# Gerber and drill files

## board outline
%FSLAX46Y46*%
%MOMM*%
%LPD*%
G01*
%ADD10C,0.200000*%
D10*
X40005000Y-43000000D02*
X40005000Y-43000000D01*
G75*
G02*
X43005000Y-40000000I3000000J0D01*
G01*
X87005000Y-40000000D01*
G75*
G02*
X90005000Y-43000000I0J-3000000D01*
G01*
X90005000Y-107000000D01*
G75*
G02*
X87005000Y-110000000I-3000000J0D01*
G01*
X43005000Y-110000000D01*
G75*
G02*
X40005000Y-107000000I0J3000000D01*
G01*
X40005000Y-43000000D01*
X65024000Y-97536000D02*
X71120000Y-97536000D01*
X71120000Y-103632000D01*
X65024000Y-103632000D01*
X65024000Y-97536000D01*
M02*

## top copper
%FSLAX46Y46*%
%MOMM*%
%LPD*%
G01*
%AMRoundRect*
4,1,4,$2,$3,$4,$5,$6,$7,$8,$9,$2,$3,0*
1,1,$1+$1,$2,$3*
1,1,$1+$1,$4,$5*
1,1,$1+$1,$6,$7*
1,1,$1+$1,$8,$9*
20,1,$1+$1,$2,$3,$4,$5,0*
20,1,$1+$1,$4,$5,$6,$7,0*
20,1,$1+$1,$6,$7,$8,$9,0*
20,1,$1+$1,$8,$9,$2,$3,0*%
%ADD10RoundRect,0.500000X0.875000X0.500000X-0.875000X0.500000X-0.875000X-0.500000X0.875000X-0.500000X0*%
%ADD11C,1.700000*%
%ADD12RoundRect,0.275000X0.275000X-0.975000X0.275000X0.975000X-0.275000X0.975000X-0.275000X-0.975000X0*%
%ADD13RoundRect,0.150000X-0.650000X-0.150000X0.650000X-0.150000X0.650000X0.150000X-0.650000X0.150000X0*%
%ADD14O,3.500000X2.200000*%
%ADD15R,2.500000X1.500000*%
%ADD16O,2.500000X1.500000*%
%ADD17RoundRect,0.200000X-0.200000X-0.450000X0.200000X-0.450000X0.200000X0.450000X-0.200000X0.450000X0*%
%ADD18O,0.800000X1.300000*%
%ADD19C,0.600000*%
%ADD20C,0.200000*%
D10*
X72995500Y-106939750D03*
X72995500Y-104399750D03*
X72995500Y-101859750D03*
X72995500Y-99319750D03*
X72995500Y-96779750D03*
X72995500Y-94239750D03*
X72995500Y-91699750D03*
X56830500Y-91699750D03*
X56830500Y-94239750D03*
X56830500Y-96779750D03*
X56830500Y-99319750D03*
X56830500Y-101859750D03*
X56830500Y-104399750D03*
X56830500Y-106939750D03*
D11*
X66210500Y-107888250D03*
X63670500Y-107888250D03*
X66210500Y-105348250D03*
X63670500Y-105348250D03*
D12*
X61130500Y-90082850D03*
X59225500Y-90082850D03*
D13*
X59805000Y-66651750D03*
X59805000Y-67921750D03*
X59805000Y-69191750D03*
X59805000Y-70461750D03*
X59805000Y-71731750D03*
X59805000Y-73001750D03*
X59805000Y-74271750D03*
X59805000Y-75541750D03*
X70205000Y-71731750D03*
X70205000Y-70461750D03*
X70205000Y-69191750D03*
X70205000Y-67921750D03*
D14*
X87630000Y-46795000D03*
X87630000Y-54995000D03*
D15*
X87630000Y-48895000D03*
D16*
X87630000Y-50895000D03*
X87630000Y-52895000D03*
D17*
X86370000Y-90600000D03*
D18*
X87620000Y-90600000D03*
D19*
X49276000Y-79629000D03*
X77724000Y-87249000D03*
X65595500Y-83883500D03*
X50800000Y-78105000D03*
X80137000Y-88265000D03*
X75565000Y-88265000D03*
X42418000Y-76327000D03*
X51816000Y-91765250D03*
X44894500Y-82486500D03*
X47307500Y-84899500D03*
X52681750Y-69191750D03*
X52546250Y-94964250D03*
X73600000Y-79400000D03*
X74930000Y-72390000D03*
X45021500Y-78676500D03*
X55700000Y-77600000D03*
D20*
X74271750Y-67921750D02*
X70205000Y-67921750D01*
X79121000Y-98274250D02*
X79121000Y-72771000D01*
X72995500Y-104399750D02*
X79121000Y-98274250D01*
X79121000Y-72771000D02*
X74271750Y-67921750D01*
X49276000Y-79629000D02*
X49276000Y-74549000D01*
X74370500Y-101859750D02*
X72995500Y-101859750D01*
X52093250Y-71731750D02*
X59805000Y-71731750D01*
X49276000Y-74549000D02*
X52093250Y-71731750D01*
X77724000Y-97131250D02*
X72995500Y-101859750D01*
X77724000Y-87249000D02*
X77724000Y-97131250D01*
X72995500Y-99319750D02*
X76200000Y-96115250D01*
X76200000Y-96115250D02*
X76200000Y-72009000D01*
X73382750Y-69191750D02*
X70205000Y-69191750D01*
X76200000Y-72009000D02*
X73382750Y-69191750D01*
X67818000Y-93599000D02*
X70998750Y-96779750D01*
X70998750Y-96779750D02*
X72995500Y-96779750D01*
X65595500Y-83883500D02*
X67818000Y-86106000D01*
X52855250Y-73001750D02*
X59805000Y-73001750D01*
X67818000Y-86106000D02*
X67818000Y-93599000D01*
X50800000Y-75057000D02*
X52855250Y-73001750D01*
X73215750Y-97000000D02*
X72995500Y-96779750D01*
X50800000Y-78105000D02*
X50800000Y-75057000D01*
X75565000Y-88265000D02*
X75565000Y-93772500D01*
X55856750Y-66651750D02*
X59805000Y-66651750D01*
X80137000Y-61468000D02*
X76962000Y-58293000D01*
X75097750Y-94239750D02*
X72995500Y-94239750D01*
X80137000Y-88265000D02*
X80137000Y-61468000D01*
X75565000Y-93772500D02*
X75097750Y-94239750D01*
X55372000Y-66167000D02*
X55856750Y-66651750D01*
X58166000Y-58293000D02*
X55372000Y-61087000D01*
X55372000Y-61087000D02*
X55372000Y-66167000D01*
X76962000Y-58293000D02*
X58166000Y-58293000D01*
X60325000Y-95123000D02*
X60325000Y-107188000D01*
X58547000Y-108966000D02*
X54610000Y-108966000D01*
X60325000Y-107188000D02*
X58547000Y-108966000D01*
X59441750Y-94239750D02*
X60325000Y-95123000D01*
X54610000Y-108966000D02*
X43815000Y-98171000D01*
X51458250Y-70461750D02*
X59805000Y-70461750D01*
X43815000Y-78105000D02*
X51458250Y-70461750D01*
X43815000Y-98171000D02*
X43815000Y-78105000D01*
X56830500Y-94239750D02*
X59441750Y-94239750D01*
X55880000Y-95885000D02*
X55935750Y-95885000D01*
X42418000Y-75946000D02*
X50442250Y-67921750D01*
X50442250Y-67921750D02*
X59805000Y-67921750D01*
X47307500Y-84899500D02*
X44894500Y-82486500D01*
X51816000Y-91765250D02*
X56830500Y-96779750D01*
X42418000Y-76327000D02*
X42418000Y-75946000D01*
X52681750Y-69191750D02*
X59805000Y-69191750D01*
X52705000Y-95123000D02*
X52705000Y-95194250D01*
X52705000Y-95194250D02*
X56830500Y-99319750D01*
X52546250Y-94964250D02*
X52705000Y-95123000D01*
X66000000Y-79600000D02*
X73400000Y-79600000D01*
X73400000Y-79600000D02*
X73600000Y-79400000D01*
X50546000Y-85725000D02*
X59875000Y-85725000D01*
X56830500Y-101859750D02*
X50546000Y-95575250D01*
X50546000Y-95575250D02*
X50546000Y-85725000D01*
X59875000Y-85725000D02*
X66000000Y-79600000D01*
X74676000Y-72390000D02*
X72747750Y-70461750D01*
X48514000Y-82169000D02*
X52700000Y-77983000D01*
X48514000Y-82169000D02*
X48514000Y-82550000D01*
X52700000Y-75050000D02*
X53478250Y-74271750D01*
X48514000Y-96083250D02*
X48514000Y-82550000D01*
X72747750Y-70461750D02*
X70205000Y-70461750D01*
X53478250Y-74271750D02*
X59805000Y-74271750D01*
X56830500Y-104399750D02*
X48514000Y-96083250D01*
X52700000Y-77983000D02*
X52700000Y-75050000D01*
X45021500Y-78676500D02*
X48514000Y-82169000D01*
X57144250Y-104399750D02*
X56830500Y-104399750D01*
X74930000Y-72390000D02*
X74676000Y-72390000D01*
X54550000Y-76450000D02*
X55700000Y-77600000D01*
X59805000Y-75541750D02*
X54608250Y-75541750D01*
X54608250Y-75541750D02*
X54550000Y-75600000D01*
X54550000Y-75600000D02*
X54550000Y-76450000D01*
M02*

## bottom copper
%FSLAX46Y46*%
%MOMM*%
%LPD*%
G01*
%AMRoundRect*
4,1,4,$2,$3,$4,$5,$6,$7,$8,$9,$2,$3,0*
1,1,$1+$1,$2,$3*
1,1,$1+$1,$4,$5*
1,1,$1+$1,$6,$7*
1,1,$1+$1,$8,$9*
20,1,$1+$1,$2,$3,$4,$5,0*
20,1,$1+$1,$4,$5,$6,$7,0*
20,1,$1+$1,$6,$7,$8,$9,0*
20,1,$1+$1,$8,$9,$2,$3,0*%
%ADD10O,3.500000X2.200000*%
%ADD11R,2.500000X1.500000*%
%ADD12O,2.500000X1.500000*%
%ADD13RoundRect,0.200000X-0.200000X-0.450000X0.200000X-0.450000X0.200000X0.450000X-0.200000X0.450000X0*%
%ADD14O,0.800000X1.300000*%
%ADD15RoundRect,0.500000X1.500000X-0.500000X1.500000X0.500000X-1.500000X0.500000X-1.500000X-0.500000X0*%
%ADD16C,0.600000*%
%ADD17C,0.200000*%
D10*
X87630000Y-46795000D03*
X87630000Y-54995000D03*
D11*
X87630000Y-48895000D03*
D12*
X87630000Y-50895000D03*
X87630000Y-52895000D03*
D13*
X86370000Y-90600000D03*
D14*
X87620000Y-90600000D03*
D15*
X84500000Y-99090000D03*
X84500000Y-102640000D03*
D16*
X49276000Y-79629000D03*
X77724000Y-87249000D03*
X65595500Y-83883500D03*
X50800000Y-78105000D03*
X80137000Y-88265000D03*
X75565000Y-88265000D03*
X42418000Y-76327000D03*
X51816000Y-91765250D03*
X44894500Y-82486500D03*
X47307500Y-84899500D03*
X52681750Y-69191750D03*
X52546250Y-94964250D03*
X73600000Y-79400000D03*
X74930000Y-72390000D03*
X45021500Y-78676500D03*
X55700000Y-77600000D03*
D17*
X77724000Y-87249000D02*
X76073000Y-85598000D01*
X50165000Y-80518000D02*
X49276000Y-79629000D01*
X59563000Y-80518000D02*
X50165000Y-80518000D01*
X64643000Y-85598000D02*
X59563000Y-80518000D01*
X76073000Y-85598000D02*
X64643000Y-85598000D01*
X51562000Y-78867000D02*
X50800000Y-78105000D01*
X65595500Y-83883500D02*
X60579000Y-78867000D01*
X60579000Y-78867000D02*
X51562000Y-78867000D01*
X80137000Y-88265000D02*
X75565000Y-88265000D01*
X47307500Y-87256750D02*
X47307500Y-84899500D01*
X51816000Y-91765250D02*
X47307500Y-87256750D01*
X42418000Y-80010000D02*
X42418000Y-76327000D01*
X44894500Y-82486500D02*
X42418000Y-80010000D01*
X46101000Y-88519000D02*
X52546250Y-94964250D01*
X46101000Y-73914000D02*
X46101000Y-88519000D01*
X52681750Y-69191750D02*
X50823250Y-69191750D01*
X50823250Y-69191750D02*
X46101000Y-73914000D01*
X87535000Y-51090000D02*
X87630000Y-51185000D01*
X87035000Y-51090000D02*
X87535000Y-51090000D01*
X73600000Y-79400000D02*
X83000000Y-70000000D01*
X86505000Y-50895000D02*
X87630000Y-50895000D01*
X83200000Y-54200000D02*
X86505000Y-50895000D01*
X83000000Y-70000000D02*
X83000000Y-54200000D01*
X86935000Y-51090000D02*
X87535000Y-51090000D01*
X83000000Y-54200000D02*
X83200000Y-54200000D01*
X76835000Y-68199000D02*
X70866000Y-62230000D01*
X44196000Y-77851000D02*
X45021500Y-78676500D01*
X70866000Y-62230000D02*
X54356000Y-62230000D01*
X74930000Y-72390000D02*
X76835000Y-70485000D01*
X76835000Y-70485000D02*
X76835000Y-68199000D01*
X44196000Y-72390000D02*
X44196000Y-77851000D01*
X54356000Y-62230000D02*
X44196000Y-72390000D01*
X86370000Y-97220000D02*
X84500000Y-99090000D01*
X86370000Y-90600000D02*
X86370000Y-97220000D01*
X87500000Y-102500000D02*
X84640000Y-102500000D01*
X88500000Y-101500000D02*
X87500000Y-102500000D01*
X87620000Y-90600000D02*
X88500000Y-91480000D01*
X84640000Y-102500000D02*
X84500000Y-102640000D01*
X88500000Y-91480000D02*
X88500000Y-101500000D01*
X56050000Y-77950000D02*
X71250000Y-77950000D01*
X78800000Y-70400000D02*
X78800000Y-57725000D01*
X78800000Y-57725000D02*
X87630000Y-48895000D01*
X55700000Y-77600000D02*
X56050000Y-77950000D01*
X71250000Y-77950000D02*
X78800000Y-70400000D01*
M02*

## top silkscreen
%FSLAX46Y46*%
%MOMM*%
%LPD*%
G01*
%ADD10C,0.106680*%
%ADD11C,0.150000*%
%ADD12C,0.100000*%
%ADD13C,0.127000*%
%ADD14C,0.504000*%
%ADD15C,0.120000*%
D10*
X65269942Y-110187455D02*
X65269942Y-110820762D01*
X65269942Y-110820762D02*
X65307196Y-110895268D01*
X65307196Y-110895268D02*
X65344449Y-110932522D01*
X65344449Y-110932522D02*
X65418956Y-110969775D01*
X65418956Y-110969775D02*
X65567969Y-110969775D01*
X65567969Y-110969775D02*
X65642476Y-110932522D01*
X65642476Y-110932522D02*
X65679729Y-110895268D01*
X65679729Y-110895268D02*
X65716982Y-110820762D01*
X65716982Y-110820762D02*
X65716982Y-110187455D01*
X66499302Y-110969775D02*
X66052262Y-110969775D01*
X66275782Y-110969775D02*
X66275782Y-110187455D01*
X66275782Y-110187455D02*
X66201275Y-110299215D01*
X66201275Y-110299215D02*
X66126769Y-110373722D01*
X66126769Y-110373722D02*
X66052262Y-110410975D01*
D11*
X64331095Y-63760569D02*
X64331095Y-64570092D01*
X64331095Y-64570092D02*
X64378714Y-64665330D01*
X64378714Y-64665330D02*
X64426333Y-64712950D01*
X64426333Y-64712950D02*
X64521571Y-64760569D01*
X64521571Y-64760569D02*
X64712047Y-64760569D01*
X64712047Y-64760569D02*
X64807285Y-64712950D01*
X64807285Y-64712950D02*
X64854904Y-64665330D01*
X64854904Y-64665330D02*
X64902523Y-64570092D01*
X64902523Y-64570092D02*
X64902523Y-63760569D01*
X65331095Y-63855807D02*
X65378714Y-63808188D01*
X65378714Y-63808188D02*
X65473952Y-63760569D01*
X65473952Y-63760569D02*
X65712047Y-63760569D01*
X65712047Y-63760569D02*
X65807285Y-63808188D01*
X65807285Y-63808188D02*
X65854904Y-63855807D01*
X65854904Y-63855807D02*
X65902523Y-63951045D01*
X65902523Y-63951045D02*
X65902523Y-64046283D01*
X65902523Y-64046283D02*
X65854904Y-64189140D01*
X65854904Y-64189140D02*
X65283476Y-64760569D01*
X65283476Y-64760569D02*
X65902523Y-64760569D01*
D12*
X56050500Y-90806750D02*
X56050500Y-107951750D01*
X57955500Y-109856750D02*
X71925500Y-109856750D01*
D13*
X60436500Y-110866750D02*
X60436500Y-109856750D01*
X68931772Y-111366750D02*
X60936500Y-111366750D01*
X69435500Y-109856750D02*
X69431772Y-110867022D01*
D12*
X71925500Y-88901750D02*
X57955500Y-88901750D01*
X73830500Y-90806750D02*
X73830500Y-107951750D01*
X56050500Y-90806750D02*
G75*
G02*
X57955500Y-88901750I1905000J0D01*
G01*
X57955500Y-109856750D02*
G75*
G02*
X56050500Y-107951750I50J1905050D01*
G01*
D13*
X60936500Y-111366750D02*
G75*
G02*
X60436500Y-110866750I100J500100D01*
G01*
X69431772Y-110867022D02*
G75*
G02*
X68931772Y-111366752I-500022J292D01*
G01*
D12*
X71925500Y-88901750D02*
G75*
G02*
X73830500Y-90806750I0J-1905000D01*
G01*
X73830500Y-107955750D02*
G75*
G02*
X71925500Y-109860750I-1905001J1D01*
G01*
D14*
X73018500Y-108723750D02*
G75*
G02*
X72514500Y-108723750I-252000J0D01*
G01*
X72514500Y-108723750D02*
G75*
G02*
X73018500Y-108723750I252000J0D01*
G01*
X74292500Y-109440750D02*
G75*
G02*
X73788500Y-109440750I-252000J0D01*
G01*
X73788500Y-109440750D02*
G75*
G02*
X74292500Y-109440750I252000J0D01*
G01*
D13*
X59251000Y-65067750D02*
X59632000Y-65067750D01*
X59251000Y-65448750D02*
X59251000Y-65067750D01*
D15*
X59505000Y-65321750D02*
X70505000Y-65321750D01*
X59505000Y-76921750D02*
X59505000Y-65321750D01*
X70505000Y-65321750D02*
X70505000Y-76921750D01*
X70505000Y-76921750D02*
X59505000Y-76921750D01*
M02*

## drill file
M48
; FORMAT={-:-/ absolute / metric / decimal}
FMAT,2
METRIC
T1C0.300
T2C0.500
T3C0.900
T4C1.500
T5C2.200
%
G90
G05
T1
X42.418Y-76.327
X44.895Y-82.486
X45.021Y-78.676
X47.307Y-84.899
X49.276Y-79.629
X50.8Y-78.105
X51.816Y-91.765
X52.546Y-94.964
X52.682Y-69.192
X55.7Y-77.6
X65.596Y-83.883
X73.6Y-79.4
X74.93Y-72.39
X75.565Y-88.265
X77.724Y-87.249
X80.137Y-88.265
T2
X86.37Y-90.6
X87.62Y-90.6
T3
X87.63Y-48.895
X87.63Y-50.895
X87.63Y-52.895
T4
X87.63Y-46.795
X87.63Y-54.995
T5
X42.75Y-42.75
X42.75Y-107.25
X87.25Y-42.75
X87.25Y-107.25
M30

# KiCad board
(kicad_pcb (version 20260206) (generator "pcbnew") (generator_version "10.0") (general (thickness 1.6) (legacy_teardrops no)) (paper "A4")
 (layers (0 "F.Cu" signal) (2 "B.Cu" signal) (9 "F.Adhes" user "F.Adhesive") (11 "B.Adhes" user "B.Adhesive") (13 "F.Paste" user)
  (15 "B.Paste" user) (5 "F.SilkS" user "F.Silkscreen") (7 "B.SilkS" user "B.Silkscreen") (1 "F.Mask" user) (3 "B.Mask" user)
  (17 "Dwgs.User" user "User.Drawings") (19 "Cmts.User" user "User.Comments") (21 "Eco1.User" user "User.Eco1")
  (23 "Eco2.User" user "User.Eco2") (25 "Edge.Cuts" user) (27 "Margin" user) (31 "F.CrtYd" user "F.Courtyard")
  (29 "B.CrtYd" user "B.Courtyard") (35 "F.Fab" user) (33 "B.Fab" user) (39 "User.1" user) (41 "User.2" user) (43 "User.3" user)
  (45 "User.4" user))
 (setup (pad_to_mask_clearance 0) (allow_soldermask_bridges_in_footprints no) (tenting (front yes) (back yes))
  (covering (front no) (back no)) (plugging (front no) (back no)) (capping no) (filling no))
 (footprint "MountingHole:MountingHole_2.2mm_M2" (layer "F.Cu") (at 87.25 42.75)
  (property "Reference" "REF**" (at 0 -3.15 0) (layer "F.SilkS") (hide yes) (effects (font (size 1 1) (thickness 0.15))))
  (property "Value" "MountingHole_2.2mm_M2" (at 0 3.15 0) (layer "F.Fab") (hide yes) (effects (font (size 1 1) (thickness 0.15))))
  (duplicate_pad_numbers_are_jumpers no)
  (pad "" np_thru_hole circle (at 0 0) (size 2.2 2.2) (drill 2.2) (layers "*.Cu" "*.Mask")))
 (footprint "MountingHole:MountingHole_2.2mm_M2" (layer "F.Cu") (at 42.75 42.75)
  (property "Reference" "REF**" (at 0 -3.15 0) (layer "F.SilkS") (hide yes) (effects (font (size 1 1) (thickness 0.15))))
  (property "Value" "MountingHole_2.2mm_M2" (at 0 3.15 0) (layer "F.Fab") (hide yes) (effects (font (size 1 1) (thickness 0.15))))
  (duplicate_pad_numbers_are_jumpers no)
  (pad "" np_thru_hole circle (at 0 0) (size 2.2 2.2) (drill 2.2) (layers "*.Cu" "*.Mask")))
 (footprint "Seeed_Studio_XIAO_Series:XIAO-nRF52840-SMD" (layer "F.Cu") (at 73.8305 88.81975 180)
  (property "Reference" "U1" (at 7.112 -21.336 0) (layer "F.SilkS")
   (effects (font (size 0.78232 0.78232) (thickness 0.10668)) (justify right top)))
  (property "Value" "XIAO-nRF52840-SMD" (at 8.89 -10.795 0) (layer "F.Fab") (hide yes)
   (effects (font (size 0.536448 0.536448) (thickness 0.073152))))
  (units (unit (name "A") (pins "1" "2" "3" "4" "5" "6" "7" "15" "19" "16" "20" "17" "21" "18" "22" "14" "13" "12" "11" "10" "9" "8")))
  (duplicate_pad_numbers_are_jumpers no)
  (fp_line (start 17.78 -1.987) (end 17.78 -19.132) (stroke (width 0.1) (type solid)) (layer "F.SilkS"))
  (fp_line (start 15.875 -21.037) (end 1.905 -21.037) (stroke (width 0.1) (type solid)) (layer "F.SilkS"))
  (fp_line (start 13.394 -22.047) (end 13.394 -21.037) (stroke (width 0.127) (type solid)) (layer "F.SilkS"))
  (fp_line (start 4.898728 -22.547) (end 12.894 -22.547) (stroke (width 0.127) (type solid)) (layer "F.SilkS"))
  (fp_line (start 4.395 -21.037) (end 4.398728 -22.047272) (stroke (width 0.127) (type solid)) (layer "F.SilkS"))
  (fp_line (start 1.905 -0.082) (end 15.875 -0.082) (stroke (width 0.1) (type solid)) (layer "F.SilkS"))
  (fp_line (start 0 -1.987) (end 0 -19.132) (stroke (width 0.1) (type solid)) (layer "F.SilkS"))
  (fp_arc (start 17.78 -1.987) (mid 17.222038 -0.639961) (end 15.875 -0.082) (stroke (width 0.1) (type solid)) (layer "F.SilkS"))
  (fp_arc (start 15.875 -21.037) (mid 17.222016 -20.479031) (end 17.78 -19.132) (stroke (width 0.1) (type solid)) (layer "F.SilkS"))
  (fp_arc (start 12.894 -22.547) (mid 13.247531 -22.400546) (end 13.394 -22.047) (stroke (width 0.127) (type default)) (layer "F.SilkS"))
  (fp_arc (start 4.398728 -22.047272) (mid 4.545276 -22.400644) (end 4.898728 -22.547) (stroke (width 0.127) (type default))
   (layer "F.SilkS"))
  (fp_arc (start 1.905 -0.082) (mid 0.557962 -0.639962) (end 0 -1.987) (stroke (width 0.1) (type solid)) (layer "F.SilkS"))
  (fp_arc (start 0 -19.136) (mid 0.557962 -20.483038) (end 1.905 -21.041) (stroke (width 0.1) (type solid)) (layer "F.SilkS"))
  (fp_circle (center 1.064 -19.904) (end 1.064 -20.158) (stroke (width 0.5) (type solid)) (fill yes) (layer "F.SilkS"))
  (fp_circle (center -0.21 -20.621) (end -0.21 -20.875) (stroke (width 0.5) (type solid)) (fill yes) (layer "F.SilkS"))
  (pad "1" smd roundrect (at 0.835 -18.12 180) (size 2.75 2) (layers "F.Cu" "F.Mask" "F.Paste") (roundrect_rratio 0.25)
   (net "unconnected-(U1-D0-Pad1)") (solder_mask_margin 0.0508) (thermal_bridge_angle 45))
  (pad "2" smd roundrect (at 0.835 -15.58 180) (size 2.75 2) (layers "F.Cu" "F.Mask" "F.Paste") (roundrect_rratio 0.25) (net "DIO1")
   (solder_mask_margin 0.0508) (thermal_bridge_angle 45))
  (pad "3" smd roundrect (at 0.835 -13.04 180) (size 2.75 2) (layers "F.Cu" "F.Mask" "F.Paste") (roundrect_rratio 0.25) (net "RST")
   (solder_mask_margin 0.0508) (thermal_bridge_angle 45))
  (pad "4" smd roundrect (at 0.835 -10.5 180) (size 2.75 2) (layers "F.Cu" "F.Mask" "F.Paste") (roundrect_rratio 0.25) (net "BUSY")
   (solder_mask_margin 0.0508) (thermal_bridge_angle 45))
  (pad "5" smd roundrect (at 0.835 -7.96 180) (size 2.75 2) (layers "F.Cu" "F.Mask" "F.Paste") (roundrect_rratio 0.25) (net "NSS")
   (solder_mask_margin 0.0508) (thermal_bridge_angle 45))
  (pad "6" smd roundrect (at 0.835 -5.42 180) (size 2.75 2) (layers "F.Cu" "F.Mask" "F.Paste") (roundrect_rratio 0.25) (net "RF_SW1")
   (solder_mask_margin 0.0508) (thermal_bridge_angle 45))
  (pad "7" smd roundrect (at 0.835 -2.88 180) (size 2.75 2) (layers "F.Cu" "F.Mask" "F.Paste") (roundrect_rratio 0.25)
   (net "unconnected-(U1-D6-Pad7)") (solder_mask_margin 0.0508) (thermal_bridge_angle 45))
  (pad "8" smd roundrect (at 17 -2.88 180) (size 2.75 2) (layers "F.Cu" "F.Mask" "F.Paste") (roundrect_rratio 0.25)
   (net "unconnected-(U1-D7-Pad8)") (solder_mask_margin 0.0508) (thermal_bridge_angle 45))
  (pad "9" smd roundrect (at 17 -5.42 180) (size 2.75 2) (layers "F.Cu" "F.Mask" "F.Paste") (roundrect_rratio 0.25) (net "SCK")
   (solder_mask_margin 0.0508) (thermal_bridge_angle 45))
  (pad "10" smd roundrect (at 17 -7.96 180) (size 2.75 2) (layers "F.Cu" "F.Mask" "F.Paste") (roundrect_rratio 0.25) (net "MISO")
   (solder_mask_margin 0.0508) (thermal_bridge_angle 45))
  (pad "11" smd roundrect (at 17 -10.5 180) (size 2.75 2) (layers "F.Cu" "F.Mask" "F.Paste") (roundrect_rratio 0.25) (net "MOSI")
   (solder_mask_margin 0.0508) (thermal_bridge_angle 45))
  (pad "12" smd roundrect (at 17 -13.04 180) (size 2.75 2) (layers "F.Cu" "F.Mask" "F.Paste") (roundrect_rratio 0.25) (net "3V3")
   (solder_mask_margin 0.0508) (thermal_bridge_angle 45))
  (pad "13" smd roundrect (at 17 -15.58 180) (size 2.75 2) (layers "F.Cu" "F.Mask" "F.Paste") (roundrect_rratio 0.25) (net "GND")
   (solder_mask_margin 0.0508) (thermal_bridge_angle 45))
  (pad "14" smd roundrect (at 17 -18.12 180) (size 2.75 2) (layers "F.Cu" "F.Mask" "F.Paste") (roundrect_rratio 0.25)
   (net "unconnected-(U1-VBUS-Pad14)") (solder_mask_margin 0.0508) (thermal_bridge_angle 45))
  (pad "15" smd circle (at 7.62 -19.0685 180) (size 1.7 1.7) (layers "F.Cu" "F.Mask" "F.Paste") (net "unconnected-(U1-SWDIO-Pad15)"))
  (pad "16" smd circle (at 10.16 -19.0685 180) (size 1.7 1.7) (layers "F.Cu" "F.Mask" "F.Paste") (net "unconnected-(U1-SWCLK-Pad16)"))
  (pad "17" smd circle (at 7.62 -16.5285 180) (size 1.7 1.7) (layers "F.Cu" "F.Mask" "F.Paste") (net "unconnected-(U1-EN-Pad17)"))
  (pad "18" smd circle (at 10.16 -16.5285 180) (size 1.7 1.7) (layers "F.Cu" "F.Mask" "F.Paste") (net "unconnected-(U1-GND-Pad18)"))
  (pad "21" smd roundrect (at 12.7 -1.2631 90) (size 2.5 1.1) (layers "F.Cu" "F.Mask" "F.Paste") (roundrect_rratio 0.25)
   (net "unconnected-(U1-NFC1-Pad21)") (thermal_bridge_angle 45))
  (pad "22" smd roundrect (at 14.605 -1.2631 90) (size 2.5 1.1) (layers "F.Cu" "F.Mask" "F.Paste") (roundrect_rratio 0.25)
   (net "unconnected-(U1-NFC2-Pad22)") (thermal_bridge_angle 45)))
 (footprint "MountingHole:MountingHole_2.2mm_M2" (layer "F.Cu") (at 42.75 107.25)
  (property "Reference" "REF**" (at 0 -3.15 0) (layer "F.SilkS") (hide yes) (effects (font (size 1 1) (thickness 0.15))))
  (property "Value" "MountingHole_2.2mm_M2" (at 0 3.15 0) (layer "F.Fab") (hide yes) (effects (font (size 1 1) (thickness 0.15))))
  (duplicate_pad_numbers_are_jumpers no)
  (pad "" np_thru_hole circle (at 0 0) (size 2.2 2.2) (drill 2.2) (layers "*.Cu" "*.Mask")))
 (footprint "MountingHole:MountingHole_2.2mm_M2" (layer "F.Cu") (at 87.25 107.25)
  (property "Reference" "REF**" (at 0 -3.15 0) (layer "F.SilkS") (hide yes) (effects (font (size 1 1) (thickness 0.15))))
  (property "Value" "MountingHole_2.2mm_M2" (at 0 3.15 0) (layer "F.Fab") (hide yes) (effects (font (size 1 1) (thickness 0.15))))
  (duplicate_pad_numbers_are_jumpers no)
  (pad "" np_thru_hole circle (at 0 0) (size 2.2 2.2) (drill 2.2) (layers "*.Cu" "*.Mask")))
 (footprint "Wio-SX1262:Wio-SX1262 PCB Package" (layer "F.Cu") (at 59.505 65.32175 -90)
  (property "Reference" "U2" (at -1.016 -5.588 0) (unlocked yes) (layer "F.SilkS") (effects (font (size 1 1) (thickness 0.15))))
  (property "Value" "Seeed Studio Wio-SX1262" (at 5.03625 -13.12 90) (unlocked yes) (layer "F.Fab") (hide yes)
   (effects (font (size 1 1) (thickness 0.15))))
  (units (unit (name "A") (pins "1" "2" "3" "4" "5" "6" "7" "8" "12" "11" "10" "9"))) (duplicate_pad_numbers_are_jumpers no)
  (fp_line (start -0.254 0.254) (end -0.254 -0.127) (stroke (width 0.127) (type default)) (layer "F.SilkS"))
  (fp_line (start 0.127 0.254) (end -0.254 0.254) (stroke (width 0.127) (type default)) (layer "F.SilkS"))
  (fp_line (start 0 0) (end 0 -11) (stroke (width 0.12) (type default)) (layer "F.SilkS"))
  (fp_line (start 11.6 0) (end 0 0) (stroke (width 0.12) (type default)) (layer "F.SilkS"))
  (fp_line (start 0 -11) (end 11.6 -11) (stroke (width 0.12) (type default)) (layer "F.SilkS"))
  (fp_line (start 11.6 -11) (end 11.6 0) (stroke (width 0.12) (type default)) (layer "F.SilkS"))
  (pad "1" smd roundrect (at 1.33 -0.3) (size 1.6 0.6) (layers "F.Cu" "F.Mask" "F.Paste") (roundrect_rratio 0.25) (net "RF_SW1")
   (thermal_bridge_angle 45))
  (pad "2" smd roundrect (at 2.6 -0.3) (size 1.6 0.6) (layers "F.Cu" "F.Mask" "F.Paste") (roundrect_rratio 0.25) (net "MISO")
   (thermal_bridge_angle 45))
  (pad "3" smd roundrect (at 3.87 -0.3) (size 1.6 0.6) (layers "F.Cu" "F.Mask" "F.Paste") (roundrect_rratio 0.25) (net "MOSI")
   (thermal_bridge_angle 45))
  (pad "4" smd roundrect (at 5.14 -0.3) (size 1.6 0.6) (layers "F.Cu" "F.Mask" "F.Paste") (roundrect_rratio 0.25) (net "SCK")
   (thermal_bridge_angle 45))
  (pad "5" smd roundrect (at 6.41 -0.3) (size 1.6 0.6) (layers "F.Cu" "F.Mask" "F.Paste") (roundrect_rratio 0.25) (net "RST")
   (thermal_bridge_angle 45))
  (pad "6" smd roundrect (at 7.68 -0.3) (size 1.6 0.6) (layers "F.Cu" "F.Mask" "F.Paste") (roundrect_rratio 0.25) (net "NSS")
   (thermal_bridge_angle 45))
  (pad "7" smd roundrect (at 8.95 -0.3) (size 1.6 0.6) (layers "F.Cu" "F.Mask" "F.Paste") (roundrect_rratio 0.25) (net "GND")
   (thermal_bridge_angle 45))
  (pad "8" smd roundrect (at 10.22 -0.3) (size 1.6 0.6) (layers "F.Cu" "F.Mask" "F.Paste") (roundrect_rratio 0.25) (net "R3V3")
   (thermal_bridge_angle 45))
  (pad "9" smd roundrect (at 6.41 -10.7) (size 1.6 0.6) (layers "F.Cu" "F.Mask" "F.Paste") (roundrect_rratio 0.25)
   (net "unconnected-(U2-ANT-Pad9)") (thermal_bridge_angle 45))
  (pad "10" smd roundrect (at 5.14 -10.7) (size 1.6 0.6) (layers "F.Cu" "F.Mask" "F.Paste") (roundrect_rratio 0.25) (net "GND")
   (thermal_bridge_angle 45))
  (pad "11" smd roundrect (at 3.87 -10.7) (size 1.6 0.6) (layers "F.Cu" "F.Mask" "F.Paste") (roundrect_rratio 0.25) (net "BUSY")
   (thermal_bridge_angle 45))
  (pad "12" smd roundrect (at 2.6 -10.7) (size 1.6 0.6) (layers "F.Cu" "F.Mask" "F.Paste") (roundrect_rratio 0.25) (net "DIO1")
   (thermal_bridge_angle 45)))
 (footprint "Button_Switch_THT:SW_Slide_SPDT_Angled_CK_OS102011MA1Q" (layer "B.Cu") (at 87.63 48.895 -90)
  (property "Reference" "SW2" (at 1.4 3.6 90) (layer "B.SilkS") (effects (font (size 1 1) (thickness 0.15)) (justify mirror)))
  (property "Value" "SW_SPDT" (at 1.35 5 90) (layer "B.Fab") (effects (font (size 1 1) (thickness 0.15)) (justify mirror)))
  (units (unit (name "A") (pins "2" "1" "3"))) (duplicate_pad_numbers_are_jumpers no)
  (pad "" thru_hole oval (at -2.1 0 270) (size 2.2 3.5) (drill 1.5) (layers "*.Cu" "*.Mask") (remove_unused_layers no))
  (pad "" thru_hole oval (at 6.1 0 270) (size 2.2 3.5) (drill 1.5) (layers "*.Cu" "*.Mask") (remove_unused_layers no))
  (pad "1" thru_hole rect (at 0 0 270) (size 1.5 2.5) (drill 0.9) (layers "*.Cu" "*.Mask") (remove_unused_layers no) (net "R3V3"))
  (pad "2" thru_hole oval (at 2 0 270) (size 1.5 2.5) (drill 0.9) (layers "*.Cu" "*.Mask") (remove_unused_layers no) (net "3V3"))
  (pad "3" thru_hole oval (at 4 0 270) (size 1.5 2.5) (drill 0.9) (layers "*.Cu" "*.Mask") (remove_unused_layers no)
   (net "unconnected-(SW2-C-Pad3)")))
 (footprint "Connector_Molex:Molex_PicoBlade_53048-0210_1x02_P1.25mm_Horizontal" (layer "B.Cu") (at 86.37 90.6)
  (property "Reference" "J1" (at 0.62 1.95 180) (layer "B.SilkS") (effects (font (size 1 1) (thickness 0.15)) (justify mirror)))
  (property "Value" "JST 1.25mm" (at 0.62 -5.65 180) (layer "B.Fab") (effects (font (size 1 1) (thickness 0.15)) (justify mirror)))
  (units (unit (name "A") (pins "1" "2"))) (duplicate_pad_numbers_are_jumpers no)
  (pad "1" thru_hole roundrect (at 0 0) (size 0.8 1.3) (drill 0.5) (layers "*.Cu" "*.Mask") (remove_unused_layers no)
   (roundrect_rratio 0.25) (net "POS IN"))
  (pad "2" thru_hole oval (at 1.25 0) (size 0.8 1.3) (drill 0.5) (layers "*.Cu" "*.Mask") (remove_unused_layers no) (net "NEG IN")))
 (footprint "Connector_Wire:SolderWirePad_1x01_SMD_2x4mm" (layer "B.Cu") (at 84.5 99.09 90)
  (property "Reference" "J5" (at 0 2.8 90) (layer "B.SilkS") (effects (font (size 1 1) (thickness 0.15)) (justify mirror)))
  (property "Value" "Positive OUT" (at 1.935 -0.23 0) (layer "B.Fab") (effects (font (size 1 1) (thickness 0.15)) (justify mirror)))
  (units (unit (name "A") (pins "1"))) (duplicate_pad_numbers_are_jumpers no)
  (pad "1" smd roundrect (at 0 0 90) (size 2 4) (layers "B.Cu" "B.Mask") (roundrect_rratio 0.25) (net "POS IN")))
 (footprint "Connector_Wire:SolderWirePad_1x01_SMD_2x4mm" (layer "B.Cu") (at 84.5 102.64 90)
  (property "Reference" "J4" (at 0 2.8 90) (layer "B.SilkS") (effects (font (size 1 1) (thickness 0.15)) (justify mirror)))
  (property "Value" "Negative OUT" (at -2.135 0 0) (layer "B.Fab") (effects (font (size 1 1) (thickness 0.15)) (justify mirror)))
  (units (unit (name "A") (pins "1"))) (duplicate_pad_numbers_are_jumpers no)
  (pad "1" smd roundrect (at 0 0 90) (size 2 4) (layers "B.Cu" "B.Mask") (roundrect_rratio 0.25) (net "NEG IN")))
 (gr_rect (start 40.005 40) (end 90.005 110) (radius 3) (stroke (width 0.2) (type solid)) (fill no) (layer "Edge.Cuts"))
 (gr_rect (start 65.024 97.536) (end 71.12 103.632) (stroke (width 0.2) (type default)) (fill no) (layer "Edge.Cuts"))
 (segment (start 74.27175 67.92175) (end 70.205 67.92175) (width 0.2) (layer "F.Cu") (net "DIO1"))
 (segment (start 79.121 98.27425) (end 79.121 72.771) (width 0.2) (layer "F.Cu") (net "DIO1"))
 (segment (start 72.9955 104.39975) (end 79.121 98.27425) (width 0.2) (layer "F.Cu") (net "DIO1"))
 (segment (start 79.121 72.771) (end 74.27175 67.92175) (width 0.2) (layer "F.Cu") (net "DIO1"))
 (segment (start 49.276 79.629) (end 49.276 74.549) (width 0.2) (layer "F.Cu") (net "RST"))
 (segment (start 74.3705 101.85975) (end 72.9955 101.85975) (width 0.2) (layer "F.Cu") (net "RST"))
 (segment (start 52.09325 71.73175) (end 59.805 71.73175) (width 0.2) (layer "F.Cu") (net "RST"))
 (segment (start 49.276 74.549) (end 52.09325 71.73175) (width 0.2) (layer "F.Cu") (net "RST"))
 (segment (start 77.724 97.13125) (end 72.9955 101.85975) (width 0.2) (layer "F.Cu") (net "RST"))
 (segment (start 77.724 87.249) (end 77.724 97.13125) (width 0.2) (layer "F.Cu") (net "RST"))
 (via (at 49.276 79.629) (size 0.6) (drill 0.3) (layers "F.Cu" "B.Cu") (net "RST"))
 (via (at 77.724 87.249) (size 0.6) (drill 0.3) (layers "F.Cu" "B.Cu") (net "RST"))
 (segment (start 77.724 87.249) (end 76.073 85.598) (width 0.2) (layer "B.Cu") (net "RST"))
 (segment (start 50.165 80.518) (end 49.276 79.629) (width 0.2) (layer "B.Cu") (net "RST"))
 (segment (start 59.563 80.518) (end 50.165 80.518) (width 0.2) (layer "B.Cu") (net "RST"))
 (segment (start 64.643 85.598) (end 59.563 80.518) (width 0.2) (layer "B.Cu") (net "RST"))
 (segment (start 76.073 85.598) (end 64.643 85.598) (width 0.2) (layer "B.Cu") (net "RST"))
 (segment (start 72.9955 99.31975) (end 76.2 96.11525) (width 0.2) (layer "F.Cu") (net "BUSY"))
 (segment (start 76.2 96.11525) (end 76.2 72.009) (width 0.2) (layer "F.Cu") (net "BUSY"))
 (segment (start 73.38275 69.19175) (end 70.205 69.19175) (width 0.2) (layer "F.Cu") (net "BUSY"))
 (segment (start 76.2 72.009) (end 73.38275 69.19175) (width 0.2) (layer "F.Cu") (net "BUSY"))
 (segment (start 67.818 93.599) (end 70.99875 96.77975) (width 0.2) (layer "F.Cu") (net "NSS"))
 (segment (start 70.99875 96.77975) (end 72.9955 96.77975) (width 0.2) (layer "F.Cu") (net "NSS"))
 (segment (start 65.5955 83.8835) (end 67.818 86.106) (width 0.2) (layer "F.Cu") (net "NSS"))
 (segment (start 52.85525 73.00175) (end 59.805 73.00175) (width 0.2) (layer "F.Cu") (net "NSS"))
 (segment (start 67.818 86.106) (end 67.818 93.599) (width 0.2) (layer "F.Cu") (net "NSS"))
 (segment (start 50.8 75.057) (end 52.85525 73.00175) (width 0.2) (layer "F.Cu") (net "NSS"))
 (segment (start 73.21575 97) (end 72.9955 96.77975) (width 0.2) (layer "F.Cu") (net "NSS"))
 (segment (start 50.8 78.105) (end 50.8 75.057) (width 0.2) (layer "F.Cu") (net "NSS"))
 (via (at 65.5955 83.8835) (size 0.6) (drill 0.3) (layers "F.Cu" "B.Cu") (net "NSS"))
 (via (at 50.8 78.105) (size 0.6) (drill 0.3) (layers "F.Cu" "B.Cu") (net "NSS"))
 (segment (start 51.562 78.867) (end 50.8 78.105) (width 0.2) (layer "B.Cu") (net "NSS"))
 (segment (start 65.5955 83.8835) (end 60.579 78.867) (width 0.2) (layer "B.Cu") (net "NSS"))
 (segment (start 60.579 78.867) (end 51.562 78.867) (width 0.2) (layer "B.Cu") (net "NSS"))
 (segment (start 75.565 88.265) (end 75.565 93.7725) (width 0.2) (layer "F.Cu") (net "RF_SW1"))
 (segment (start 55.85675 66.65175) (end 59.805 66.65175) (width 0.2) (layer "F.Cu") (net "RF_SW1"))
 (segment (start 80.137 61.468) (end 76.962 58.293) (width 0.2) (layer "F.Cu") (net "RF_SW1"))
 (segment (start 75.09775 94.23975) (end 72.9955 94.23975) (width 0.2) (layer "F.Cu") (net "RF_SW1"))
 (segment (start 80.137 88.265) (end 80.137 61.468) (width 0.2) (layer "F.Cu") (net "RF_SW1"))
 (segment (start 75.565 93.7725) (end 75.09775 94.23975) (width 0.2) (layer "F.Cu") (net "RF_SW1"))
 (segment (start 55.372 66.167) (end 55.85675 66.65175) (width 0.2) (layer "F.Cu") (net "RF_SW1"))
 (segment (start 58.166 58.293) (end 55.372 61.087) (width 0.2) (layer "F.Cu") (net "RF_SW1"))
 (segment (start 55.372 61.087) (end 55.372 66.167) (width 0.2) (layer "F.Cu") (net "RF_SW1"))
 (segment (start 76.962 58.293) (end 58.166 58.293) (width 0.2) (layer "F.Cu") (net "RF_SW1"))
 (via (at 80.137 88.265) (size 0.6) (drill 0.3) (layers "F.Cu" "B.Cu") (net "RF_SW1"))
 (via (at 75.565 88.265) (size 0.6) (drill 0.3) (layers "F.Cu" "B.Cu") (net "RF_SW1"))
 (segment (start 80.137 88.265) (end 75.565 88.265) (width 0.2) (layer "B.Cu") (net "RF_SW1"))
 (segment (start 60.325 95.123) (end 60.325 107.188) (width 0.2) (layer "F.Cu") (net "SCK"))
 (segment (start 58.547 108.966) (end 54.61 108.966) (width 0.2) (layer "F.Cu") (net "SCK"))
 (segment (start 60.325 107.188) (end 58.547 108.966) (width 0.2) (layer "F.Cu") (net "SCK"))
 (segment (start 59.44175 94.23975) (end 60.325 95.123) (width 0.2) (layer "F.Cu") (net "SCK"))
 (segment (start 54.61 108.966) (end 43.815 98.171) (width 0.2) (layer "F.Cu") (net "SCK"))
 (segment (start 51.45825 70.46175) (end 59.805 70.46175) (width 0.2) (layer "F.Cu") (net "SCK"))
 (segment (start 43.815 78.105) (end 51.45825 70.46175) (width 0.2) (layer "F.Cu") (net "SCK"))
 (segment (start 43.815 98.171) (end 43.815 78.105) (width 0.2) (layer "F.Cu") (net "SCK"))
 (segment (start 56.8305 94.23975) (end 59.44175 94.23975) (width 0.2) (layer "F.Cu") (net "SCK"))
 (segment (start 55.88 95.885) (end 55.93575 95.885) (width 0.2) (layer "F.Cu") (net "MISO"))
 (segment (start 42.418 75.946) (end 50.44225 67.92175) (width 0.2) (layer "F.Cu") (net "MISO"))
 (segment (start 50.44225 67.92175) (end 59.805 67.92175) (width 0.2) (layer "F.Cu") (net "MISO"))
 (segment (start 47.3075 84.8995) (end 44.8945 82.4865) (width 0.2) (layer "F.Cu") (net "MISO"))
 (segment (start 51.816 91.76525) (end 56.8305 96.77975) (width 0.2) (layer "F.Cu") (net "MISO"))
 (segment (start 42.418 76.327) (end 42.418 75.946) (width 0.2) (layer "F.Cu") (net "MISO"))
 (via (at 42.418 76.327) (size 0.6) (drill 0.3) (layers "F.Cu" "B.Cu") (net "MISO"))
 (via (at 51.816 91.76525) (size 0.6) (drill 0.3) (layers "F.Cu" "B.Cu") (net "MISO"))
 (via (at 44.8945 82.4865) (size 0.6) (drill 0.3) (layers "F.Cu" "B.Cu") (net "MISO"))
 (via (at 47.3075 84.8995) (size 0.6) (drill 0.3) (layers "F.Cu" "B.Cu") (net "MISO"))
 (segment (start 47.3075 87.25675) (end 47.3075 84.8995) (width 0.2) (layer "B.Cu") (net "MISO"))
 (segment (start 51.816 91.76525) (end 47.3075 87.25675) (width 0.2) (layer "B.Cu") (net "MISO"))
 (segment (start 42.418 80.01) (end 42.418 76.327) (width 0.2) (layer "B.Cu") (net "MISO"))
 (segment (start 44.8945 82.4865) (end 42.418 80.01) (width 0.2) (layer "B.Cu") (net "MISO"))
 (segment (start 52.68175 69.19175) (end 59.805 69.19175) (width 0.2) (layer "F.Cu") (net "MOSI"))
 (segment (start 52.705 95.123) (end 52.705 95.19425) (width 0.2) (layer "F.Cu") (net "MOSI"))
 (segment (start 52.705 95.19425) (end 56.8305 99.31975) (width 0.2) (layer "F.Cu") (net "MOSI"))
 (segment (start 52.54625 94.96425) (end 52.705 95.123) (width 0.2) (layer "F.Cu") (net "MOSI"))
 (via (at 52.68175 69.19175) (size 0.6) (drill 0.3) (layers "F.Cu" "B.Cu") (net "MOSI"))
 (via (at 52.54625 94.96425) (size 0.6) (drill 0.3) (layers "F.Cu" "B.Cu") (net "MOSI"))
 (segment (start 46.101 88.519) (end 52.54625 94.96425) (width 0.2) (layer "B.Cu") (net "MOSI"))
 (segment (start 46.101 73.914) (end 46.101 88.519) (width 0.2) (layer "B.Cu") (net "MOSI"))
 (segment (start 52.68175 69.19175) (end 50.82325 69.19175) (width 0.2) (layer "B.Cu") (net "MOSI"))
 (segment (start 50.82325 69.19175) (end 46.101 73.914) (width 0.2) (layer "B.Cu") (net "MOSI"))
 (segment (start 66 79.6) (end 73.4 79.6) (width 0.2) (layer "F.Cu") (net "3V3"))
 (segment (start 73.4 79.6) (end 73.6 79.4) (width 0.2) (layer "F.Cu") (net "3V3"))
 (segment (start 50.546 85.725) (end 59.875 85.725) (width 0.2) (layer "F.Cu") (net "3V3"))
 (segment (start 56.8305 101.85975) (end 50.546 95.57525) (width 0.2) (layer "F.Cu") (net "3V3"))
 (segment (start 50.546 95.57525) (end 50.546 85.725) (width 0.2) (layer "F.Cu") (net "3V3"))
 (segment (start 59.875 85.725) (end 66 79.6) (width 0.2) (layer "F.Cu") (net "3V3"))
 (via (at 73.6 79.4) (size 0.6) (drill 0.3) (layers "F.Cu" "B.Cu") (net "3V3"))
 (segment (start 87.535 51.09) (end 87.63 51.185) (width 0.2) (layer "B.Cu") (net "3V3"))
 (segment (start 87.035 51.09) (end 87.535 51.09) (width 0.2) (layer "B.Cu") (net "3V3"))
 (segment (start 73.6 79.4) (end 83 70) (width 0.2) (layer "B.Cu") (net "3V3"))
 (segment (start 86.505 50.895) (end 87.63 50.895) (width 0.2) (layer "B.Cu") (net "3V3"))
 (segment (start 83.2 54.2) (end 86.505 50.895) (width 0.2) (layer "B.Cu") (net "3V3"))
 (segment (start 83 70) (end 83 54.2) (width 0.2) (layer "B.Cu") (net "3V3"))
 (segment (start 86.935 51.09) (end 87.535 51.09) (width 0.2) (layer "B.Cu") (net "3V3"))
 (segment (start 83 54.2) (end 83.2 54.2) (width 0.2) (layer "B.Cu") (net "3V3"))
 (segment (start 74.676 72.39) (end 72.74775 70.46175) (width 0.2) (layer "F.Cu") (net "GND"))
 (segment (start 48.514 82.169) (end 52.7 77.983) (width 0.2) (layer "F.Cu") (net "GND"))
 (segment (start 48.514 82.169) (end 48.514 82.55) (width 0.2) (layer "F.Cu") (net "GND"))
 (segment (start 52.7 75.05) (end 53.47825 74.27175) (width 0.2) (layer "F.Cu") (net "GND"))
 (segment (start 48.514 96.08325) (end 48.514 82.55) (width 0.2) (layer "F.Cu") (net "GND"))
 (segment (start 72.74775 70.46175) (end 70.205 70.46175) (width 0.2) (layer "F.Cu") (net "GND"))
 (segment (start 53.47825 74.27175) (end 59.805 74.27175) (width 0.2) (layer "F.Cu") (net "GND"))
 (segment (start 56.8305 104.39975) (end 48.514 96.08325) (width 0.2) (layer "F.Cu") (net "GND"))
 (segment (start 52.7 77.983) (end 52.7 75.05) (width 0.2) (layer "F.Cu") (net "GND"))
 (segment (start 45.0215 78.6765) (end 48.514 82.169) (width 0.2) (layer "F.Cu") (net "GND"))
 (segment (start 57.14425 104.39975) (end 56.8305 104.39975) (width 0.2) (layer "F.Cu") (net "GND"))
 (segment (start 74.93 72.39) (end 74.676 72.39) (width 0.2) (layer "F.Cu") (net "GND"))
 (via (at 74.93 72.39) (size 0.6) (drill 0.3) (layers "F.Cu" "B.Cu") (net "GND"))
 (via (at 45.0215 78.6765) (size 0.6) (drill 0.3) (layers "F.Cu" "B.Cu") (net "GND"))
 (segment (start 76.835 68.199) (end 70.866 62.23) (width 0.2) (layer "B.Cu") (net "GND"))
 (segment (start 44.196 77.851) (end 45.0215 78.6765) (width 0.2) (layer "B.Cu") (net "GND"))
 (segment (start 70.866 62.23) (end 54.356 62.23) (width 0.2) (layer "B.Cu") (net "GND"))
 (segment (start 74.93 72.39) (end 76.835 70.485) (width 0.2) (layer "B.Cu") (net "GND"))
 (segment (start 76.835 70.485) (end 76.835 68.199) (width 0.2) (layer "B.Cu") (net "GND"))
 (segment (start 44.196 72.39) (end 44.196 77.851) (width 0.2) (layer "B.Cu") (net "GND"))
 (segment (start 54.356 62.23) (end 44.196 72.39) (width 0.2) (layer "B.Cu") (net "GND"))
 (segment (start 86.37 97.22) (end 84.5 99.09) (width 0.2) (layer "B.Cu") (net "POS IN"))
 (segment (start 86.37 90.6) (end 86.37 97.22) (width 0.2) (layer "B.Cu") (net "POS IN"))
 (segment (start 87.5 102.5) (end 84.64 102.5) (width 0.2) (layer "B.Cu") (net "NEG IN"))
 (segment (start 88.5 101.5) (end 87.5 102.5) (width 0.2) (layer "B.Cu") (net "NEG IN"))
 (segment (start 87.62 90.6) (end 88.5 91.48) (width 0.2) (layer "B.Cu") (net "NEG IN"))
 (segment (start 84.64 102.5) (end 84.5 102.64) (width 0.2) (layer "B.Cu") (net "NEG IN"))
 (segment (start 88.5 91.48) (end 88.5 101.5) (width 0.2) (layer "B.Cu") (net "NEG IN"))
 (segment (start 54.55 76.45) (end 55.7 77.6) (width 0.2) (layer "F.Cu") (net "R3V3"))
 (segment (start 59.805 75.54175) (end 54.60825 75.54175) (width 0.2) (layer "F.Cu") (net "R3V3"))
 (segment (start 54.60825 75.54175) (end 54.55 75.6) (width 0.2) (layer "F.Cu") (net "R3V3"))
 (segment (start 54.55 75.6) (end 54.55 76.45) (width 0.2) (layer "F.Cu") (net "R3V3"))
 (via (at 55.7 77.6) (size 0.6) (drill 0.3) (layers "F.Cu" "B.Cu") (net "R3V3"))
 (segment (start 56.05 77.95) (end 71.25 77.95) (width 0.2) (layer "B.Cu") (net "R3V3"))
 (segment (start 78.8 70.4) (end 78.8 57.725) (width 0.2) (layer "B.Cu") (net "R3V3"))
 (segment (start 78.8 57.725) (end 87.63 48.895) (width 0.2) (layer "B.Cu") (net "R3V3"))
 (segment (start 55.7 77.6) (end 56.05 77.95) (width 0.2) (layer "B.Cu") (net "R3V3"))
 (segment (start 71.25 77.95) (end 78.8 70.4) (width 0.2) (layer "B.Cu") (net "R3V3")))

